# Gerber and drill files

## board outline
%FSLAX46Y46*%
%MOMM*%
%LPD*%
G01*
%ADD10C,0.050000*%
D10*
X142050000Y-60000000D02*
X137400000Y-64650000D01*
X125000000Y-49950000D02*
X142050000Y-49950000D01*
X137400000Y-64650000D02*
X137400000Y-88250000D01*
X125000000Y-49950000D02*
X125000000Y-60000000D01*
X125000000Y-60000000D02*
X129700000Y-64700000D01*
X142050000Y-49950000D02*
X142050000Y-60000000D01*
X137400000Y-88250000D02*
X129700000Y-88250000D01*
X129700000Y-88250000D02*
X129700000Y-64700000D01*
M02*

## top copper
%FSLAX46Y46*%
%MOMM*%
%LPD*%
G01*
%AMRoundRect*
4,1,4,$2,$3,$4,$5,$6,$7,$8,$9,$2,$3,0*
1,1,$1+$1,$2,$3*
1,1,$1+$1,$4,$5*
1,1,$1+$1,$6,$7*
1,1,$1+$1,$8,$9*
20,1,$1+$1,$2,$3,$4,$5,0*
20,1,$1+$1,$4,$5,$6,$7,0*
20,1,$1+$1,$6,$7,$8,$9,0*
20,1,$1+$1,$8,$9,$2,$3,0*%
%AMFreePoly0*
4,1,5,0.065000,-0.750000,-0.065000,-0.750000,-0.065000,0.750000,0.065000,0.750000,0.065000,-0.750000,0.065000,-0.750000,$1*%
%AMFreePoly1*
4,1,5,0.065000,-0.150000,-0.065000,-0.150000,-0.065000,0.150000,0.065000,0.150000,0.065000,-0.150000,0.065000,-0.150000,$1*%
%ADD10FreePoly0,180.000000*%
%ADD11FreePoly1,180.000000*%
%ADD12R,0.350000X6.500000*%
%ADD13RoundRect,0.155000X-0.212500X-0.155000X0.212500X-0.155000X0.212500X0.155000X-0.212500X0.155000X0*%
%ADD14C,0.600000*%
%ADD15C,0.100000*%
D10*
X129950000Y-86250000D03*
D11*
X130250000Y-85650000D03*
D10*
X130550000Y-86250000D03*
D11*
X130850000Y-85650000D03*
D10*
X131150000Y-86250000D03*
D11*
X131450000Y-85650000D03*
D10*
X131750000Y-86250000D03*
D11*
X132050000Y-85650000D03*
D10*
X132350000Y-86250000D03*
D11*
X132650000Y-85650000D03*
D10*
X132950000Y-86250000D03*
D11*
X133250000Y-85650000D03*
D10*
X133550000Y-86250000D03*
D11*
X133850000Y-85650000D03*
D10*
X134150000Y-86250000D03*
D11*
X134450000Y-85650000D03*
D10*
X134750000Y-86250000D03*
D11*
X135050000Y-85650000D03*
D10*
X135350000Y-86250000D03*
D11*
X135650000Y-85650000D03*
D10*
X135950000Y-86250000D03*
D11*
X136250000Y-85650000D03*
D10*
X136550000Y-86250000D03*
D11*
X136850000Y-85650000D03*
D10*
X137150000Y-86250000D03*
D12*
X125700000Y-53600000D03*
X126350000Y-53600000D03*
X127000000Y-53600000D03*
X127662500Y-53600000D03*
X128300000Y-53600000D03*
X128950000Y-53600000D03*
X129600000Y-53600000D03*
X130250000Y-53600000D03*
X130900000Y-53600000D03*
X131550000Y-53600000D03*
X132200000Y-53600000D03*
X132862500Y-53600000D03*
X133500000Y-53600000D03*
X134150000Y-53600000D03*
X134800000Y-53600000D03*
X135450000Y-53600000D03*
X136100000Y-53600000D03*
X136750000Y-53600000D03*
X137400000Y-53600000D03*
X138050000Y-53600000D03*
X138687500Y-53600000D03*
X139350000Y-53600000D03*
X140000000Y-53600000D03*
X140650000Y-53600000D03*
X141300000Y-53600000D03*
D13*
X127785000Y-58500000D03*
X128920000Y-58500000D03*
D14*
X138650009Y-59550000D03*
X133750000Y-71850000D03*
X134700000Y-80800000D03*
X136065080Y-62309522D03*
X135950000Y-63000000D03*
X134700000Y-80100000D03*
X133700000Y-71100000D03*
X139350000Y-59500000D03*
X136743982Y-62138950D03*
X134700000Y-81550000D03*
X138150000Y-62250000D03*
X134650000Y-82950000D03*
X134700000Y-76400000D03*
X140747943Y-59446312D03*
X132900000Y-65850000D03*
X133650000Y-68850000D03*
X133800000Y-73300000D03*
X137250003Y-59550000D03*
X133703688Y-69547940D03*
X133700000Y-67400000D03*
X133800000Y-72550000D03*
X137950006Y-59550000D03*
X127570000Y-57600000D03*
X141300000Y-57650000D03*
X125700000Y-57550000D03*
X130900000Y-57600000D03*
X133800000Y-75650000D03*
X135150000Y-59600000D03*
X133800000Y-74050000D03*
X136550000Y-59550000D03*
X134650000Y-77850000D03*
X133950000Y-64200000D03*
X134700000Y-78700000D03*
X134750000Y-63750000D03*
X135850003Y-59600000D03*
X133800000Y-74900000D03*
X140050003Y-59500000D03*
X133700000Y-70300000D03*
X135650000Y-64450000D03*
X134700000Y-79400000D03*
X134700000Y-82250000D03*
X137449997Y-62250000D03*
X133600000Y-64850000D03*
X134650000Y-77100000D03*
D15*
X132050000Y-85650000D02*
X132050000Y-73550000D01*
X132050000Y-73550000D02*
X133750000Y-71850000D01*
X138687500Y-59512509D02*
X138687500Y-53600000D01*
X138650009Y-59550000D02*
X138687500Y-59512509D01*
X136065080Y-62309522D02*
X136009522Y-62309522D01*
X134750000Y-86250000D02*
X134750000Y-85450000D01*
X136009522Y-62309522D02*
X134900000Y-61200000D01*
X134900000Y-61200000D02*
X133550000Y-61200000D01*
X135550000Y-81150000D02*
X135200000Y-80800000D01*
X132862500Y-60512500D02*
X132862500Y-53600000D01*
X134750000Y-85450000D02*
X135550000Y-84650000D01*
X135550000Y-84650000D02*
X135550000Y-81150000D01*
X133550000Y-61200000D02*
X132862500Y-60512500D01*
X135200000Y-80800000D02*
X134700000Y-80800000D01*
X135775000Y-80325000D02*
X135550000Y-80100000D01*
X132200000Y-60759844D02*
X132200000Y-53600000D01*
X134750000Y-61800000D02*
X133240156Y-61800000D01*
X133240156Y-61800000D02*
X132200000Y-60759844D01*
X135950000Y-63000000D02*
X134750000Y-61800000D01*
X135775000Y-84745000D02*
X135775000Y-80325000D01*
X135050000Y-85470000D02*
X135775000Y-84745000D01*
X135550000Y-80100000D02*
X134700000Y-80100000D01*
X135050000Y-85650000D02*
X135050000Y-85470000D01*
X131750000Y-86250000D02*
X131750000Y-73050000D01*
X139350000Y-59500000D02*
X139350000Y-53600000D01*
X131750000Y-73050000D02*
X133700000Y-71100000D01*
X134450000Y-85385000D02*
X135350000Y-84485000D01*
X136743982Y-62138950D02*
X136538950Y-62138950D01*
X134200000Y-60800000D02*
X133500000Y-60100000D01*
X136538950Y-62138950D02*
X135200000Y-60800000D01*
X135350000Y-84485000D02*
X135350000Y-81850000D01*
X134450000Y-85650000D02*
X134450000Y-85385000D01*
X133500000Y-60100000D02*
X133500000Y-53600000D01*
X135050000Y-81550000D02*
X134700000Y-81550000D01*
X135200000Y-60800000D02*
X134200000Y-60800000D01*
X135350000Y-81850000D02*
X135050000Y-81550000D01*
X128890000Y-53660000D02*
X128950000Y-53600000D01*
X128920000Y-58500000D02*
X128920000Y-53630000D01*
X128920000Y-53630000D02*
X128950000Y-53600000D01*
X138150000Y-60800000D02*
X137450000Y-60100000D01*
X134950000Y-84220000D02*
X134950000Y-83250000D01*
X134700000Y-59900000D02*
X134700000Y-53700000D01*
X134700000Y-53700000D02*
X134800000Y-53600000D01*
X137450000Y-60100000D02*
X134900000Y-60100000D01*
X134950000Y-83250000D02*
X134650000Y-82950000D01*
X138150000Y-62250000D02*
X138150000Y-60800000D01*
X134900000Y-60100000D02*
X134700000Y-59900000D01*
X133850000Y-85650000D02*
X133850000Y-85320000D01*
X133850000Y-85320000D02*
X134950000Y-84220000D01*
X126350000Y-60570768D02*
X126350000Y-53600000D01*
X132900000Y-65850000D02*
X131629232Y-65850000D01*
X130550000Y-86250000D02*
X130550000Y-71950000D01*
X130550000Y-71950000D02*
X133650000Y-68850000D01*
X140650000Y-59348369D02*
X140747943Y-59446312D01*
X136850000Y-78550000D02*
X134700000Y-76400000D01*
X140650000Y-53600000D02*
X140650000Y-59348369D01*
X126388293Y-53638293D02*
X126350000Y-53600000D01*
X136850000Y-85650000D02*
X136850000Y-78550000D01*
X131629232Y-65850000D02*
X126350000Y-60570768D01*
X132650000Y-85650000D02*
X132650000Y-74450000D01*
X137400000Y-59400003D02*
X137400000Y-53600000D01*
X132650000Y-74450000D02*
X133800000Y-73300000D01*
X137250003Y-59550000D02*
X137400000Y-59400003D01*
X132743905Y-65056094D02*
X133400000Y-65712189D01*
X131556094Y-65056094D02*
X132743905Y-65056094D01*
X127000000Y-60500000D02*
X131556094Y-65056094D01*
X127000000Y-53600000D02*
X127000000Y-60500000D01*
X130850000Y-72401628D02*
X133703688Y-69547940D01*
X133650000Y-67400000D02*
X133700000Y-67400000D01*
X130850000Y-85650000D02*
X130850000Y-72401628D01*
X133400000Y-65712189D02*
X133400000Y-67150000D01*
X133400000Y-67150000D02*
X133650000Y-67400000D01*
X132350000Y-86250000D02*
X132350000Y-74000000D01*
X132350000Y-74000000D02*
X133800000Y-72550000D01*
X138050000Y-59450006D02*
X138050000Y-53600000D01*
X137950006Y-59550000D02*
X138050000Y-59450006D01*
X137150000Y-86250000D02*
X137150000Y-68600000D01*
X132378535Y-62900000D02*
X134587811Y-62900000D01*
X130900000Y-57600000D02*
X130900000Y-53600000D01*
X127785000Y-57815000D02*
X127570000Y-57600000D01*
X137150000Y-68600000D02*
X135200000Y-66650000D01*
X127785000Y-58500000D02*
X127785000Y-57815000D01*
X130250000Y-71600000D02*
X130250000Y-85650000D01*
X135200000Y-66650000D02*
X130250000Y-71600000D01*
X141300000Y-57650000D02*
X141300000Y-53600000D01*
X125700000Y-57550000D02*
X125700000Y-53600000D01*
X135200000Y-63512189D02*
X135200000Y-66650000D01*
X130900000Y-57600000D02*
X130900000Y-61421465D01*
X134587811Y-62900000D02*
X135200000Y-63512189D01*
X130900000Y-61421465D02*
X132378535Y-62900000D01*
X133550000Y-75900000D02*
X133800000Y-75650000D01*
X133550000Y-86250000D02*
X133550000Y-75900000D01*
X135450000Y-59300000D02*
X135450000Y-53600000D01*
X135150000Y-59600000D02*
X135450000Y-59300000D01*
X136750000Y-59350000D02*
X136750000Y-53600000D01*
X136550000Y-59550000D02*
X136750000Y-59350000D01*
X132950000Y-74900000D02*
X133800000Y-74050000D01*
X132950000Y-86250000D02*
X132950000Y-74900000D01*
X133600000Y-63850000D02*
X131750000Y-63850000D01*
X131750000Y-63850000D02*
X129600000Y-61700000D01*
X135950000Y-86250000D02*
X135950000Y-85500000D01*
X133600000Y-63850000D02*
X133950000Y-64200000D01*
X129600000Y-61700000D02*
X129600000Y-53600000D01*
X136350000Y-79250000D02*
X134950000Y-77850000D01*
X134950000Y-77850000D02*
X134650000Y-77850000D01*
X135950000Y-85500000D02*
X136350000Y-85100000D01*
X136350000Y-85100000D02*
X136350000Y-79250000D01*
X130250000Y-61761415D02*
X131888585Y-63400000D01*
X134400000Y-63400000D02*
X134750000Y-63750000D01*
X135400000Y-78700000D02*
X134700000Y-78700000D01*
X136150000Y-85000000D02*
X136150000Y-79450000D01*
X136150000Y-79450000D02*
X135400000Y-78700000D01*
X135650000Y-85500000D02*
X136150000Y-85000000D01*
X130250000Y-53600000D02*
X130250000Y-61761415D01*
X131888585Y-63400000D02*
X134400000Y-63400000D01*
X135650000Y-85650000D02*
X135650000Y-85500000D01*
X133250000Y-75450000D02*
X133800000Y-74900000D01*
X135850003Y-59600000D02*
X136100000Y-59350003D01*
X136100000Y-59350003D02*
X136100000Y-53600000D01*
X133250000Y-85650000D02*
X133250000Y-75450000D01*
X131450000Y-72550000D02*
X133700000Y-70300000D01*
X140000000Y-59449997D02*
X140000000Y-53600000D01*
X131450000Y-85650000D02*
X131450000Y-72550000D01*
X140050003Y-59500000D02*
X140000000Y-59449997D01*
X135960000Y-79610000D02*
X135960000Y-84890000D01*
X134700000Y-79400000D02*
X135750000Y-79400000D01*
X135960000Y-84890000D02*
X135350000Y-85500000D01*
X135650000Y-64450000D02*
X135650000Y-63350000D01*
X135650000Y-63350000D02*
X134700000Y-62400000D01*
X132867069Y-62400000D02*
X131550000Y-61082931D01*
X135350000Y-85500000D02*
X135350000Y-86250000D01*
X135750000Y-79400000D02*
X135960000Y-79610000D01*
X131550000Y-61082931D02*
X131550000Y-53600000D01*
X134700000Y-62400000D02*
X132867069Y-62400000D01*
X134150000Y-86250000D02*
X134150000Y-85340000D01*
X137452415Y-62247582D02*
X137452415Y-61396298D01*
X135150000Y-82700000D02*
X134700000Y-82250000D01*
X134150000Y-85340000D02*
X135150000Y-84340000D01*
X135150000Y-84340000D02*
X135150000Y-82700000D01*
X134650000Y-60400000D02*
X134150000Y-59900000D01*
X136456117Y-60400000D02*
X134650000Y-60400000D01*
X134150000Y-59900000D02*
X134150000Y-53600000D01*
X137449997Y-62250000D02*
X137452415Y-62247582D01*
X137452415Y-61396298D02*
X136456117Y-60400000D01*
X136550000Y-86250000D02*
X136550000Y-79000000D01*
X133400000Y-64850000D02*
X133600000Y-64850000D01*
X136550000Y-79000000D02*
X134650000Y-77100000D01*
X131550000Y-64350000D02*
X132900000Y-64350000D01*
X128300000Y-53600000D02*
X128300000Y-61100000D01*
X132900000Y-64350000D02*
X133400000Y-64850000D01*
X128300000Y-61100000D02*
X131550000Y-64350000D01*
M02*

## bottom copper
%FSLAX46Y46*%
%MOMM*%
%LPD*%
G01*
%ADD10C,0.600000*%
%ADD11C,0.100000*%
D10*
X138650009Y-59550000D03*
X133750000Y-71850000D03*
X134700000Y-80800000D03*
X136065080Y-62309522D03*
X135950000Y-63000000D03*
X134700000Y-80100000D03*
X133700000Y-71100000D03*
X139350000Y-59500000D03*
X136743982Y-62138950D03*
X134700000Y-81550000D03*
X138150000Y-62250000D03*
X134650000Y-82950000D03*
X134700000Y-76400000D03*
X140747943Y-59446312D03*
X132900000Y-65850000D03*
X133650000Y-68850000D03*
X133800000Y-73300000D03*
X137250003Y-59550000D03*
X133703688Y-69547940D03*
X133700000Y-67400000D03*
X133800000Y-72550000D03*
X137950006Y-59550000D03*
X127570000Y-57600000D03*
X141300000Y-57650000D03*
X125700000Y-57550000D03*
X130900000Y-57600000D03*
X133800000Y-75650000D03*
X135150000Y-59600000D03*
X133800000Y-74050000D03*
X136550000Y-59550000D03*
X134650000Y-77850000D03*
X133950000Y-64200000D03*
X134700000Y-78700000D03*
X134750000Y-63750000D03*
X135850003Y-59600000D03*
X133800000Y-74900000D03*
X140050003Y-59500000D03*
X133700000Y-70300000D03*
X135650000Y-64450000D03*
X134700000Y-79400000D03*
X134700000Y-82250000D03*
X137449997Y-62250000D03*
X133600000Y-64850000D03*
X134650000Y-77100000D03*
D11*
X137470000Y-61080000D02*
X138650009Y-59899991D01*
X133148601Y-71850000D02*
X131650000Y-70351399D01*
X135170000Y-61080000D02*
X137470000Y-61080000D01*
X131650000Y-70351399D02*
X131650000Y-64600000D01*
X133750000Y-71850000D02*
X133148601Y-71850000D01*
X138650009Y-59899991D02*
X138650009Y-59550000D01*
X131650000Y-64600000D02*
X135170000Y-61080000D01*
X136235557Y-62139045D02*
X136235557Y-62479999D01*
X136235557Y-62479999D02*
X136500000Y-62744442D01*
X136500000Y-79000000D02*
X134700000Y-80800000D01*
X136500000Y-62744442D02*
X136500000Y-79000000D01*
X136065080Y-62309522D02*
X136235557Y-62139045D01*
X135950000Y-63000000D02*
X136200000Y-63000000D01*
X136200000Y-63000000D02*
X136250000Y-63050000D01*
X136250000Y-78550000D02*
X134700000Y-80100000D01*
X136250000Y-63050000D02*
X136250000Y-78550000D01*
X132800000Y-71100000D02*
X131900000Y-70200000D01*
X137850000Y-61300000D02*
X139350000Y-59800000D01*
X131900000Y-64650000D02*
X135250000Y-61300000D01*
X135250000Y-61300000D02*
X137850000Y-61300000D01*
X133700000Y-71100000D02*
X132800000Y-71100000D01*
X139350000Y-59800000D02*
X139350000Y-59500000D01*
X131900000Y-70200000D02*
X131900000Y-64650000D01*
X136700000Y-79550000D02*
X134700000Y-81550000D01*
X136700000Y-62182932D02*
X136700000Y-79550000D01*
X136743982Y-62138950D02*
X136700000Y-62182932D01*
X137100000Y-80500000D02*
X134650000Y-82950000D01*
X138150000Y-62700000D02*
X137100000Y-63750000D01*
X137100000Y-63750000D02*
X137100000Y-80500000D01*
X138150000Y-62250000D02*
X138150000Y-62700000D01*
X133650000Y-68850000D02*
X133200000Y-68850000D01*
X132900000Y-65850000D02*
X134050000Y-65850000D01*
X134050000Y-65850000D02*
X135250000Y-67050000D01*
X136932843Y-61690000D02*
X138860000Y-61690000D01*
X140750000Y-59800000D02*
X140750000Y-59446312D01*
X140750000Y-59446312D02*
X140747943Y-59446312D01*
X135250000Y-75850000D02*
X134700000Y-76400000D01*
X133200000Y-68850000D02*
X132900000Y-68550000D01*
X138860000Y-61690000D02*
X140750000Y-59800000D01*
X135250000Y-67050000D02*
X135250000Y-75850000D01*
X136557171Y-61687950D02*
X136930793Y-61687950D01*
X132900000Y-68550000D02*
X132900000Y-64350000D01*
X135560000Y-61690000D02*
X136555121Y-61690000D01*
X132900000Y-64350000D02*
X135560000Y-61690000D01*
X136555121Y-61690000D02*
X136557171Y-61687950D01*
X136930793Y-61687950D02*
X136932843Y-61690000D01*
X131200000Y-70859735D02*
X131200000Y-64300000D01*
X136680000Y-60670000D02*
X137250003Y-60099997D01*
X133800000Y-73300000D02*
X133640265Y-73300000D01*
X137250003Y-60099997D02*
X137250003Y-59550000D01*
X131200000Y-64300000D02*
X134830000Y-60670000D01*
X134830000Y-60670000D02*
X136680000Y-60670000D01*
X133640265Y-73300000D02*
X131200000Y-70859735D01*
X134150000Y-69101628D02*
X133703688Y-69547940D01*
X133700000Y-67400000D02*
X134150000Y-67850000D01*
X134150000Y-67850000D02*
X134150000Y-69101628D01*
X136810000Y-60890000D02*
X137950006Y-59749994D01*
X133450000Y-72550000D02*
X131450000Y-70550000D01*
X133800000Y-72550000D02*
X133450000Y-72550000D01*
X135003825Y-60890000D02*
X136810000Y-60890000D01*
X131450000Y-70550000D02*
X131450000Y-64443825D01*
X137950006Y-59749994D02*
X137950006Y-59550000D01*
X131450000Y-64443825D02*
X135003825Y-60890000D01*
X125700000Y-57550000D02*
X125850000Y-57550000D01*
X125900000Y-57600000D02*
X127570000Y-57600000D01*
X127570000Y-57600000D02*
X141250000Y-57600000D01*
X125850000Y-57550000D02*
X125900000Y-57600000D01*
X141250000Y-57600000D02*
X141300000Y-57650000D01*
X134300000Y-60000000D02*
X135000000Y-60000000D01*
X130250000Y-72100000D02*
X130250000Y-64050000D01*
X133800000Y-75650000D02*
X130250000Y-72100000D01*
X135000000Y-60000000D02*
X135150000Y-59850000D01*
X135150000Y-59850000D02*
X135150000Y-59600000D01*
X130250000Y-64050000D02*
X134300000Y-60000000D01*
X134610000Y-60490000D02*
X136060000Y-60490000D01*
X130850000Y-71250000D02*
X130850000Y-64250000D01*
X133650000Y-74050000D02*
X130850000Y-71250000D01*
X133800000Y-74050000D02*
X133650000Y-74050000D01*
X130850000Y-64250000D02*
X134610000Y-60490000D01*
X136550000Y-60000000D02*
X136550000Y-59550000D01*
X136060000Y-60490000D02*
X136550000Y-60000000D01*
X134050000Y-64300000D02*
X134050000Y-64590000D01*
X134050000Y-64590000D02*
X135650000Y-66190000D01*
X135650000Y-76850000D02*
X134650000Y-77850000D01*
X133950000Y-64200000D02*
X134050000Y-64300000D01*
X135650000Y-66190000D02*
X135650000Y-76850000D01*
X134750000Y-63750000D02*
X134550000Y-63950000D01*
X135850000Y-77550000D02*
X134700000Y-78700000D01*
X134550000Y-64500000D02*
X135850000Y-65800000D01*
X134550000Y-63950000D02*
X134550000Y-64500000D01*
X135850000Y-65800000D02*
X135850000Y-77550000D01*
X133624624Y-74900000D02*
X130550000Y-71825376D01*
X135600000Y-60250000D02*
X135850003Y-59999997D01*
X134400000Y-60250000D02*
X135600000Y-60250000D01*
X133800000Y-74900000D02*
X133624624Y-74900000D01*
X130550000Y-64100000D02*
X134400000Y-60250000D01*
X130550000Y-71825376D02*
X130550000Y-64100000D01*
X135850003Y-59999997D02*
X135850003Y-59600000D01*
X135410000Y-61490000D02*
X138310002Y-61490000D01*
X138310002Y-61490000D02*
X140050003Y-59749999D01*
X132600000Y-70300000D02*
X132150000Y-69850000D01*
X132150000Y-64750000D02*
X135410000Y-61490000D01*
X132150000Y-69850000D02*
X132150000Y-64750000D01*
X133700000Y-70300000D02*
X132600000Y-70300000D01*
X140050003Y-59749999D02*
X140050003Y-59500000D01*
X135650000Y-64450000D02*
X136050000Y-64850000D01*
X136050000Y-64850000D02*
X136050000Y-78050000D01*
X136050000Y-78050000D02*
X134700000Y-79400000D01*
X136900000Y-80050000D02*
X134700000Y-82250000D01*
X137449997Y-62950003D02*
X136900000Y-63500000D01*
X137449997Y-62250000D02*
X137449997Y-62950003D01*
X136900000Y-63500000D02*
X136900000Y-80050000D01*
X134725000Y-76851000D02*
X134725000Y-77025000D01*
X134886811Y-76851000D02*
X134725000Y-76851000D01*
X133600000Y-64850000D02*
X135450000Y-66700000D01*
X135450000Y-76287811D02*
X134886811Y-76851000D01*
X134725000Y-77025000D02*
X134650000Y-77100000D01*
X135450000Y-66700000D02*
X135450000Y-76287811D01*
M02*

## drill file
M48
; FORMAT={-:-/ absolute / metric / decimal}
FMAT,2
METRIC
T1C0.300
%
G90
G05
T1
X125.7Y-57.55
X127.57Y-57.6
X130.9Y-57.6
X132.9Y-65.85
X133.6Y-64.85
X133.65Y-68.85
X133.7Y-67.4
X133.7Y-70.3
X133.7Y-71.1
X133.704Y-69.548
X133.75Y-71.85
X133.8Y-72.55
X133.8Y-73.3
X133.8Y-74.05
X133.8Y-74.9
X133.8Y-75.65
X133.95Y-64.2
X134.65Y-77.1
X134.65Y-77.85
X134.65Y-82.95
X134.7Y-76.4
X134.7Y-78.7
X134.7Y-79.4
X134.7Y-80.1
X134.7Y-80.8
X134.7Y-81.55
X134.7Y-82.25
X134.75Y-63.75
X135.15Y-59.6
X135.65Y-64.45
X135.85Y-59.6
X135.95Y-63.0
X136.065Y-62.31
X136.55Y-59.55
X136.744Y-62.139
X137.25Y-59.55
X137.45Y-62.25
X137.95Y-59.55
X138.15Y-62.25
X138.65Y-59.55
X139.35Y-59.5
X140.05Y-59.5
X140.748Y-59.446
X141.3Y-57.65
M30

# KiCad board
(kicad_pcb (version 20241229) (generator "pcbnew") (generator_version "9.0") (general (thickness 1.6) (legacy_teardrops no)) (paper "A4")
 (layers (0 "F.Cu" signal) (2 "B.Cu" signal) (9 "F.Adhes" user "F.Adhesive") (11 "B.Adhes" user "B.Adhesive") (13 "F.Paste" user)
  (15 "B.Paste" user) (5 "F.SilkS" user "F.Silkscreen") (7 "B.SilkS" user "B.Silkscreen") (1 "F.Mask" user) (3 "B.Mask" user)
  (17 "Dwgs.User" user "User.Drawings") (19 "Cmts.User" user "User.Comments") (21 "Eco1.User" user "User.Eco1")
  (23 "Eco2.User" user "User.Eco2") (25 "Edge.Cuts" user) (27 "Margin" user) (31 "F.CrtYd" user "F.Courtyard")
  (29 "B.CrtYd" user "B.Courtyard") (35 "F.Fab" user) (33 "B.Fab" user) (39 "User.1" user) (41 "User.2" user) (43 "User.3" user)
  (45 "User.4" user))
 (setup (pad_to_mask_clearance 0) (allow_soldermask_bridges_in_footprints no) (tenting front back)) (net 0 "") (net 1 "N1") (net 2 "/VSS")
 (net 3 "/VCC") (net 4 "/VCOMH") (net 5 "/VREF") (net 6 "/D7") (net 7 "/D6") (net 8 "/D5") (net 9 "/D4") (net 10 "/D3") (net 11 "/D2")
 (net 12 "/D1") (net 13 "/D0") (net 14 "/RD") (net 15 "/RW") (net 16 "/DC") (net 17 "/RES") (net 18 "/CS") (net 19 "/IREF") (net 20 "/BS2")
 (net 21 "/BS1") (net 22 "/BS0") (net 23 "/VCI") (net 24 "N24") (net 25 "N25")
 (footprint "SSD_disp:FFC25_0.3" (layer "F.Cu") (at 137.15 86.25 180)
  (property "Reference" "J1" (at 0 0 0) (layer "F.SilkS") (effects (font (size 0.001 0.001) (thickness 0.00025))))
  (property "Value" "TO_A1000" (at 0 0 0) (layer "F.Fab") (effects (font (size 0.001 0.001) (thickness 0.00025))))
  (pad "1" smd custom (at 7.2 0 180) (size 0.13 1.5) (layers "F.Cu" "F.Mask" "F.Paste") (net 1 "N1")
   (options (clearance outline) (anchor rect)) (primitives))
  (pad "2" smd custom (at 6.9 0.6 180) (size 0.13 0.3) (layers "F.Cu" "F.Mask" "F.Paste") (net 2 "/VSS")
   (options (clearance outline) (anchor rect)) (primitives))
  (pad "3" smd custom (at 6.6 0 180) (size 0.13 1.5) (layers "F.Cu" "F.Mask" "F.Paste") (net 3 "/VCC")
   (options (clearance outline) (anchor rect)) (primitives))
  (pad "4" smd custom (at 6.3 0.6 180) (size 0.13 0.3) (layers "F.Cu" "F.Mask" "F.Paste") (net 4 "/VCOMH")
   (options (clearance outline) (anchor rect)) (primitives))
  (pad "5" smd custom (at 6 0 180) (size 0.13 1.5) (layers "F.Cu" "F.Mask" "F.Paste") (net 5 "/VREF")
   (options (clearance outline) (anchor rect)) (primitives))
  (pad "6" smd custom (at 5.7 0.6 180) (size 0.13 0.3) (layers "F.Cu" "F.Mask" "F.Paste") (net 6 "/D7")
   (options (clearance outline) (anchor rect)) (primitives))
  (pad "7" smd custom (at 5.4 0 180) (size 0.13 1.5) (layers "F.Cu" "F.Mask" "F.Paste") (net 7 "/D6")
   (options (clearance outline) (anchor rect)) (primitives))
  (pad "8" smd custom (at 5.1 0.6 180) (size 0.13 0.3) (layers "F.Cu" "F.Mask" "F.Paste") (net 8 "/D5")
   (options (clearance outline) (anchor rect)) (primitives))
  (pad "9" smd custom (at 4.8 0 180) (size 0.13 1.5) (layers "F.Cu" "F.Mask" "F.Paste") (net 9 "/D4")
   (options (clearance outline) (anchor rect)) (primitives))
  (pad "10" smd custom (at 4.5 0.6 180) (size 0.13 0.3) (layers "F.Cu" "F.Mask" "F.Paste") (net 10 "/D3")
   (options (clearance outline) (anchor rect)) (primitives))
  (pad "11" smd custom (at 4.2 0 180) (size 0.13 1.5) (layers "F.Cu" "F.Mask" "F.Paste") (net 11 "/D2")
   (options (clearance outline) (anchor rect)) (primitives))
  (pad "12" smd custom (at 3.9 0.6 180) (size 0.13 0.3) (layers "F.Cu" "F.Mask" "F.Paste") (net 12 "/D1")
   (options (clearance outline) (anchor rect)) (primitives))
  (pad "13" smd custom (at 3.6 0 180) (size 0.13 1.5) (layers "F.Cu" "F.Mask" "F.Paste") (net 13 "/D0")
   (options (clearance outline) (anchor rect)) (primitives))
  (pad "14" smd custom (at 3.3 0.6 180) (size 0.13 0.3) (layers "F.Cu" "F.Mask" "F.Paste") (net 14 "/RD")
   (options (clearance outline) (anchor rect)) (primitives))
  (pad "15" smd custom (at 3 0 180) (size 0.13 1.5) (layers "F.Cu" "F.Mask" "F.Paste") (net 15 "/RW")
   (options (clearance outline) (anchor rect)) (primitives))
  (pad "16" smd custom (at 2.7 0.6 180) (size 0.13 0.3) (layers "F.Cu" "F.Mask" "F.Paste") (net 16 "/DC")
   (options (clearance outline) (anchor rect)) (primitives))
  (pad "17" smd custom (at 2.4 0 180) (size 0.13 1.5) (layers "F.Cu" "F.Mask" "F.Paste") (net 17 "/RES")
   (options (clearance outline) (anchor rect)) (primitives))
  (pad "18" smd custom (at 2.1 0.6 180) (size 0.13 0.3) (layers "F.Cu" "F.Mask" "F.Paste") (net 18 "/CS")
   (options (clearance outline) (anchor rect)) (primitives))
  (pad "19" smd custom (at 1.8 0 180) (size 0.13 1.5) (layers "F.Cu" "F.Mask" "F.Paste") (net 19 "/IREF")
   (options (clearance outline) (anchor rect)) (primitives))
  (pad "20" smd custom (at 1.5 0.6 180) (size 0.13 0.3) (layers "F.Cu" "F.Mask" "F.Paste") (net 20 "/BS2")
   (options (clearance outline) (anchor rect)) (primitives))
  (pad "21" smd custom (at 1.2 0 180) (size 0.13 1.5) (layers "F.Cu" "F.Mask" "F.Paste") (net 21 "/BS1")
   (options (clearance outline) (anchor rect)) (primitives))
  (pad "22" smd custom (at 0.9 0.6 180) (size 0.13 0.3) (layers "F.Cu" "F.Mask" "F.Paste") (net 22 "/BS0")
   (options (clearance outline) (anchor rect)) (primitives))
  (pad "23" smd custom (at 0.6 0 180) (size 0.13 1.5) (layers "F.Cu" "F.Mask" "F.Paste") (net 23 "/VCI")
   (options (clearance outline) (anchor rect)) (primitives))
  (pad "24" smd custom (at 0.3 0.6 180) (size 0.13 0.3) (layers "F.Cu" "F.Mask" "F.Paste") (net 3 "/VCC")
   (options (clearance outline) (anchor rect)) (primitives))
  (pad "25" smd custom (at 0 0 180) (size 0.13 1.5) (layers "F.Cu" "F.Mask" "F.Paste") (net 2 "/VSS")
   (options (clearance outline) (anchor rect)) (primitives)))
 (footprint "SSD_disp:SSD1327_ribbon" (layer "F.Cu") (at 135.85 51.35)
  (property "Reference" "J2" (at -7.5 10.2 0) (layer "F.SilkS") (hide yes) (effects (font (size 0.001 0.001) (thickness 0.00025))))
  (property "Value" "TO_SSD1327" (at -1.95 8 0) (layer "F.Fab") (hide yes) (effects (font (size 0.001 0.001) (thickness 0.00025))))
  (pad "1" smd rect (at -10.15 2.25) (size 0.35 6.5) (layers "F.Cu" "F.Mask" "F.Paste") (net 2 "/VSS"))
  (pad "2" smd rect (at -9.5 2.25) (size 0.35 6.5) (layers "F.Cu" "F.Mask" "F.Paste") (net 3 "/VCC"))
  (pad "3" smd rect (at -8.85 2.25) (size 0.35 6.5) (layers "F.Cu" "F.Mask" "F.Paste") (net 4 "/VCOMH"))
  (pad "4" smd rect (at -8.1875 2.25) (size 0.35 6.5) (layers "F.Cu" "F.Mask" "F.Paste") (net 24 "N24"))
  (pad "5" smd rect (at -7.55 2.25) (size 0.35 6.5) (layers "F.Cu" "F.Mask" "F.Paste") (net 23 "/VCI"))
  (pad "6" smd rect (at -6.9 2.25) (size 0.35 6.5) (layers "F.Cu" "F.Mask" "F.Paste") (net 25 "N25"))
  (pad "7" smd rect (at -6.25 2.25) (size 0.35 6.5) (layers "F.Cu" "F.Mask" "F.Paste") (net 21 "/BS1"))
  (pad "8" smd rect (at -5.6 2.25) (size 0.35 6.5) (layers "F.Cu" "F.Mask" "F.Paste") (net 20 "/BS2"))
  (pad "9" smd rect (at -4.95 2.25) (size 0.35 6.5) (layers "F.Cu" "F.Mask" "F.Paste") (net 2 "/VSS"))
  (pad "10" smd rect (at -4.3 2.25) (size 0.35 6.5) (layers "F.Cu" "F.Mask" "F.Paste") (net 19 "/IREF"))
  (pad "11" smd rect (at -3.65 2.25) (size 0.35 6.5) (layers "F.Cu" "F.Mask" "F.Paste") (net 18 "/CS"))
  (pad "12" smd rect (at -2.9875 2.25) (size 0.35 6.5) (layers "F.Cu" "F.Mask" "F.Paste") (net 17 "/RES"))
  (pad "13" smd rect (at -2.35 2.25) (size 0.35 6.5) (layers "F.Cu" "F.Mask" "F.Paste") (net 16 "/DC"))
  (pad "14" smd rect (at -1.7 2.25) (size 0.35 6.5) (layers "F.Cu" "F.Mask" "F.Paste") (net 15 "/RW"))
  (pad "15" smd rect (at -1.05 2.25) (size 0.35 6.5) (layers "F.Cu" "F.Mask" "F.Paste") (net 14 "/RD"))
  (pad "16" smd rect (at -0.4 2.25) (size 0.35 6.5) (layers "F.Cu" "F.Mask" "F.Paste") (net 13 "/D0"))
  (pad "17" smd rect (at 0.25 2.25) (size 0.35 6.5) (layers "F.Cu" "F.Mask" "F.Paste") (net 12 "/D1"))
  (pad "18" smd rect (at 0.9 2.25) (size 0.35 6.5) (layers "F.Cu" "F.Mask" "F.Paste") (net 11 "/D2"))
  (pad "19" smd rect (at 1.55 2.25) (size 0.35 6.5) (layers "F.Cu" "F.Mask" "F.Paste") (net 10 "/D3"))
  (pad "20" smd rect (at 2.2 2.25) (size 0.35 6.5) (layers "F.Cu" "F.Mask" "F.Paste") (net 9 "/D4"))
  (pad "21" smd rect (at 2.8375 2.25) (size 0.35 6.5) (layers "F.Cu" "F.Mask" "F.Paste") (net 8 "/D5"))
  (pad "22" smd rect (at 3.5 2.25) (size 0.35 6.5) (layers "F.Cu" "F.Mask" "F.Paste") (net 7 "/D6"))
  (pad "23" smd rect (at 4.15 2.25) (size 0.35 6.5) (layers "F.Cu" "F.Mask" "F.Paste") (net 6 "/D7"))
  (pad "24" smd rect (at 4.8 2.25) (size 0.35 6.5) (layers "F.Cu" "F.Mask" "F.Paste") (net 3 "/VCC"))
  (pad "25" smd rect (at 5.45 2.25) (size 0.35 6.5) (layers "F.Cu" "F.Mask" "F.Paste") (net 2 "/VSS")))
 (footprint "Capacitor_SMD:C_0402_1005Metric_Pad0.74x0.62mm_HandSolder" (layer "F.Cu") (at 128.3525 58.5)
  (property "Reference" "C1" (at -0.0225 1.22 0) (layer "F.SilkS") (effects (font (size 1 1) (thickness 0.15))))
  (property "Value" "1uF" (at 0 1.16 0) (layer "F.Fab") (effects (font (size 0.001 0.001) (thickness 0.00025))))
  (pad "1" smd roundrect (at -0.5675 0) (size 0.735 0.62) (layers "F.Cu" "F.Mask" "F.Paste") (roundrect_rratio 0.25) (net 2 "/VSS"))
  (pad "2" smd roundrect (at 0.5675 0) (size 0.735 0.62) (layers "F.Cu" "F.Mask" "F.Paste") (roundrect_rratio 0.25) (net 25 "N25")))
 (gr_line (start 142.05 60) (end 137.4 64.65) (stroke (width 0.05) (type solid)) (layer "Edge.Cuts"))
 (gr_line (start 125 49.95) (end 142.05 49.95) (stroke (width 0.05) (type default)) (layer "Edge.Cuts"))
 (gr_line (start 137.4 64.65) (end 137.4 88.25) (stroke (width 0.05) (type solid)) (layer "Edge.Cuts"))
 (gr_line (start 125 49.95) (end 125 60) (stroke (width 0.05) (type solid)) (layer "Edge.Cuts"))
 (gr_line (start 125 60) (end 129.7 64.7) (stroke (width 0.05) (type solid)) (layer "Edge.Cuts"))
 (gr_line (start 142.05 49.95) (end 142.05 60) (stroke (width 0.05) (type solid)) (layer "Edge.Cuts"))
 (gr_line (start 137.4 88.25) (end 129.7 88.25) (stroke (width 0.05) (type default)) (layer "Edge.Cuts"))
 (gr_line (start 129.7 88.25) (end 129.7 64.7) (stroke (width 0.05) (type solid)) (layer "Edge.Cuts"))
 (segment (start 132.05 85.65) (end 132.05 73.55) (width 0.1) (layer "F.Cu") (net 8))
 (segment (start 132.05 73.55) (end 133.75 71.85) (width 0.1) (layer "F.Cu") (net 8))
 (segment (start 138.6875 59.512509) (end 138.6875 53.6) (width 0.1) (layer "F.Cu") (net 8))
 (segment (start 138.650009 59.55) (end 138.6875 59.512509) (width 0.1) (layer "F.Cu") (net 8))
 (via (at 138.650009 59.55) (size 0.6) (drill 0.3) (layers "F.Cu" "B.Cu") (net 8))
 (via (at 133.75 71.85) (size 0.6) (drill 0.3) (layers "F.Cu" "B.Cu") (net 8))
 (segment (start 137.47 61.08) (end 138.650009 59.899991) (width 0.1) (layer "B.Cu") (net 8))
 (segment (start 133.148601 71.85) (end 131.65 70.351399) (width 0.1) (layer "B.Cu") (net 8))
 (segment (start 135.17 61.08) (end 137.47 61.08) (width 0.1) (layer "B.Cu") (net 8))
 (segment (start 131.65 70.351399) (end 131.65 64.6) (width 0.1) (layer "B.Cu") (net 8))
 (segment (start 133.75 71.85) (end 133.148601 71.85) (width 0.1) (layer "B.Cu") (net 8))
 (segment (start 138.650009 59.899991) (end 138.650009 59.55) (width 0.1) (layer "B.Cu") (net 8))
 (segment (start 131.65 64.6) (end 135.17 61.08) (width 0.1) (layer "B.Cu") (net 8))
 (segment (start 136.06508 62.309522) (end 136.009522 62.309522) (width 0.1) (layer "F.Cu") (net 17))
 (segment (start 134.75 86.25) (end 134.75 85.45) (width 0.1) (layer "F.Cu") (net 17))
 (segment (start 136.009522 62.309522) (end 134.9 61.2) (width 0.1) (layer "F.Cu") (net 17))
 (segment (start 134.9 61.2) (end 133.55 61.2) (width 0.1) (layer "F.Cu") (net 17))
 (segment (start 135.55 81.15) (end 135.2 80.8) (width 0.1) (layer "F.Cu") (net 17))
 (segment (start 132.8625 60.5125) (end 132.8625 53.6) (width 0.1) (layer "F.Cu") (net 17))
 (segment (start 134.75 85.45) (end 135.55 84.65) (width 0.1) (layer "F.Cu") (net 17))
 (segment (start 135.55 84.65) (end 135.55 81.15) (width 0.1) (layer "F.Cu") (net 17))
 (segment (start 133.55 61.2) (end 132.8625 60.5125) (width 0.1) (layer "F.Cu") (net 17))
 (segment (start 135.2 80.8) (end 134.7 80.8) (width 0.1) (layer "F.Cu") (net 17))
 (via (at 134.7 80.8) (size 0.6) (drill 0.3) (layers "F.Cu" "B.Cu") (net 17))
 (via (at 136.06508 62.309522) (size 0.6) (drill 0.3) (layers "F.Cu" "B.Cu") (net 17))
 (segment (start 136.235557 62.139045) (end 136.235557 62.479999) (width 0.1) (layer "B.Cu") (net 17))
 (segment (start 136.235557 62.479999) (end 136.5 62.744442) (width 0.1) (layer "B.Cu") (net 17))
 (segment (start 136.5 79) (end 134.7 80.8) (width 0.1) (layer "B.Cu") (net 17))
 (segment (start 136.5 62.744442) (end 136.5 79) (width 0.1) (layer "B.Cu") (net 17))
 (segment (start 136.06508 62.309522) (end 136.235557 62.139045) (width 0.1) (layer "B.Cu") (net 17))
 (segment (start 135.775 80.325) (end 135.55 80.1) (width 0.1) (layer "F.Cu") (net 18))
 (segment (start 132.2 60.759844) (end 132.2 53.6) (width 0.1) (layer "F.Cu") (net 18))
 (segment (start 134.75 61.8) (end 133.240156 61.8) (width 0.1) (layer "F.Cu") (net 18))
 (segment (start 133.240156 61.8) (end 132.2 60.759844) (width 0.1) (layer "F.Cu") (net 18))
 (segment (start 135.95 63) (end 134.75 61.8) (width 0.1) (layer "F.Cu") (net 18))
 (segment (start 135.775 84.745) (end 135.775 80.325) (width 0.1) (layer "F.Cu") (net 18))
 (segment (start 135.05 85.47) (end 135.775 84.745) (width 0.1) (layer "F.Cu") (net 18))
 (segment (start 135.55 80.1) (end 134.7 80.1) (width 0.1) (layer "F.Cu") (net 18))
 (segment (start 135.05 85.65) (end 135.05 85.47) (width 0.1) (layer "F.Cu") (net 18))
 (via (at 135.95 63) (size 0.6) (drill 0.3) (layers "F.Cu" "B.Cu") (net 18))
 (via (at 134.7 80.1) (size 0.6) (drill 0.3) (layers "F.Cu" "B.Cu") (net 18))
 (segment (start 135.95 63) (end 136.2 63) (width 0.1) (layer "B.Cu") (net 18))
 (segment (start 136.2 63) (end 136.25 63.05) (width 0.1) (layer "B.Cu") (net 18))
 (segment (start 136.25 78.55) (end 134.7 80.1) (width 0.1) (layer "B.Cu") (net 18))
 (segment (start 136.25 63.05) (end 136.25 78.55) (width 0.1) (layer "B.Cu") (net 18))
 (segment (start 131.75 86.25) (end 131.75 73.05) (width 0.1) (layer "F.Cu") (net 7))
 (segment (start 139.35 59.5) (end 139.35 53.6) (width 0.1) (layer "F.Cu") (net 7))
 (segment (start 131.75 73.05) (end 133.7 71.1) (width 0.1) (layer "F.Cu") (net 7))
 (via (at 133.7 71.1) (size 0.6) (drill 0.3) (layers "F.Cu" "B.Cu") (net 7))
 (via (at 139.35 59.5) (size 0.6) (drill 0.3) (layers "F.Cu" "B.Cu") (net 7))
 (segment (start 132.8 71.1) (end 131.9 70.2) (width 0.1) (layer "B.Cu") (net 7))
 (segment (start 137.85 61.3) (end 139.35 59.8) (width 0.1) (layer "B.Cu") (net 7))
 (segment (start 131.9 64.65) (end 135.25 61.3) (width 0.1) (layer "B.Cu") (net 7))
 (segment (start 135.25 61.3) (end 137.85 61.3) (width 0.1) (layer "B.Cu") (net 7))
 (segment (start 133.7 71.1) (end 132.8 71.1) (width 0.1) (layer "B.Cu") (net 7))
 (segment (start 139.35 59.8) (end 139.35 59.5) (width 0.1) (layer "B.Cu") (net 7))
 (segment (start 131.9 70.2) (end 131.9 64.65) (width 0.1) (layer "B.Cu") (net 7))
 (segment (start 134.45 85.385) (end 135.35 84.485) (width 0.1) (layer "F.Cu") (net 16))
 (segment (start 136.743982 62.13895) (end 136.53895 62.13895) (width 0.1) (layer "F.Cu") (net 16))
 (segment (start 134.2 60.8) (end 133.5 60.1) (width 0.1) (layer "F.Cu") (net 16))
 (segment (start 136.53895 62.13895) (end 135.2 60.8) (width 0.1) (layer "F.Cu") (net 16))
 (segment (start 135.35 84.485) (end 135.35 81.85) (width 0.1) (layer "F.Cu") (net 16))
 (segment (start 134.45 85.65) (end 134.45 85.385) (width 0.1) (layer "F.Cu") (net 16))
 (segment (start 133.5 60.1) (end 133.5 53.6) (width 0.1) (layer "F.Cu") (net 16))
 (segment (start 135.05 81.55) (end 134.7 81.55) (width 0.1) (layer "F.Cu") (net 16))
 (segment (start 135.2 60.8) (end 134.2 60.8) (width 0.1) (layer "F.Cu") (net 16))
 (segment (start 135.35 81.85) (end 135.05 81.55) (width 0.1) (layer "F.Cu") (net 16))
 (via (at 136.743982 62.13895) (size 0.6) (drill 0.3) (layers "F.Cu" "B.Cu") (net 16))
 (via (at 134.7 81.55) (size 0.6) (drill 0.3) (layers "F.Cu" "B.Cu") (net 16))
 (segment (start 136.7 79.55) (end 134.7 81.55) (width 0.1) (layer "B.Cu") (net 16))
 (segment (start 136.7 62.182932) (end 136.7 79.55) (width 0.1) (layer "B.Cu") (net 16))
 (segment (start 136.743982 62.13895) (end 136.7 62.182932) (width 0.1) (layer "B.Cu") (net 16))
 (segment (start 128.89 53.66) (end 128.95 53.6) (width 0.1) (layer "F.Cu") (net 25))
 (segment (start 128.92 58.5) (end 128.92 53.63) (width 0.1) (layer "F.Cu") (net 25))
 (segment (start 128.92 53.63) (end 128.95 53.6) (width 0.1) (layer "F.Cu") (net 25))
 (segment (start 138.15 60.8) (end 137.45 60.1) (width 0.1) (layer "F.Cu") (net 14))
 (segment (start 134.95 84.22) (end 134.95 83.25) (width 0.1) (layer "F.Cu") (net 14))
 (segment (start 134.7 59.9) (end 134.7 53.7) (width 0.1) (layer "F.Cu") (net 14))
 (segment (start 134.7 53.7) (end 134.8 53.6) (width 0.1) (layer "F.Cu") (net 14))
 (segment (start 137.45 60.1) (end 134.9 60.1) (width 0.1) (layer "F.Cu") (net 14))
 (segment (start 134.95 83.25) (end 134.65 82.95) (width 0.1) (layer "F.Cu") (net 14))
 (segment (start 138.15 62.25) (end 138.15 60.8) (width 0.1) (layer "F.Cu") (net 14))
 (segment (start 134.9 60.1) (end 134.7 59.9) (width 0.1) (layer "F.Cu") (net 14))
 (segment (start 133.85 85.65) (end 133.85 85.32) (width 0.1) (layer "F.Cu") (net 14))
 (segment (start 133.85 85.32) (end 134.95 84.22) (width 0.1) (layer "F.Cu") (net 14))
 (via (at 138.15 62.25) (size 0.6) (drill 0.3) (layers "F.Cu" "B.Cu") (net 14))
 (via (at 134.65 82.95) (size 0.6) (drill 0.3) (layers "F.Cu" "B.Cu") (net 14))
 (segment (start 137.1 80.5) (end 134.65 82.95) (width 0.1) (layer "B.Cu") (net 14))
 (segment (start 138.15 62.7) (end 137.1 63.75) (width 0.1) (layer "B.Cu") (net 14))
 (segment (start 137.1 63.75) (end 137.1 80.5) (width 0.1) (layer "B.Cu") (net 14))
 (segment (start 138.15 62.25) (end 138.15 62.7) (width 0.1) (layer "B.Cu") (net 14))
 (segment (start 126.35 60.570768) (end 126.35 53.6) (width 0.1) (layer "F.Cu") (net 3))
 (segment (start 132.9 65.85) (end 131.629232 65.85) (width 0.1) (layer "F.Cu") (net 3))
 (segment (start 130.55 86.25) (end 130.55 71.95) (width 0.1) (layer "F.Cu") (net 3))
 (segment (start 130.55 71.95) (end 133.65 68.85) (width 0.1) (layer "F.Cu") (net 3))
 (segment (start 140.65 59.348369) (end 140.747943 59.446312) (width 0.1) (layer "F.Cu") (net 3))
 (segment (start 136.85 78.55) (end 134.7 76.4) (width 0.1) (layer "F.Cu") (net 3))
 (segment (start 140.65 53.6) (end 140.65 59.348369) (width 0.1) (layer "F.Cu") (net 3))
 (segment (start 126.388293 53.638293) (end 126.35 53.6) (width 0.1) (layer "F.Cu") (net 3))
 (segment (start 136.85 85.65) (end 136.85 78.55) (width 0.1) (layer "F.Cu") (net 3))
 (segment (start 131.629232 65.85) (end 126.35 60.570768) (width 0.1) (layer "F.Cu") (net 3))
 (via (at 134.7 76.4) (size 0.6) (drill 0.3) (layers "F.Cu" "B.Cu") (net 3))
 (via (at 140.747943 59.446312) (size 0.6) (drill 0.3) (layers "F.Cu" "B.Cu") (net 3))
 (via (at 132.9 65.85) (size 0.6) (drill 0.3) (layers "F.Cu" "B.Cu") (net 3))
 (via (at 133.65 68.85) (size 0.6) (drill 0.3) (layers "F.Cu" "B.Cu") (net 3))
 (segment (start 133.65 68.85) (end 133.2 68.85) (width 0.1) (layer "B.Cu") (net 3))
 (segment (start 132.9 65.85) (end 134.05 65.85) (width 0.1) (layer "B.Cu") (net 3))
 (segment (start 134.05 65.85) (end 135.25 67.05) (width 0.1) (layer "B.Cu") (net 3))
 (segment (start 136.932843 61.69) (end 138.86 61.69) (width 0.1) (layer "B.Cu") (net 3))
 (segment (start 140.75 59.8) (end 140.75 59.446312) (width 0.1) (layer "B.Cu") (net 3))
 (segment (start 140.75 59.446312) (end 140.747943 59.446312) (width 0.1) (layer "B.Cu") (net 3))
 (segment (start 135.25 75.85) (end 134.7 76.4) (width 0.1) (layer "B.Cu") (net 3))
 (segment (start 133.2 68.85) (end 132.9 68.55) (width 0.1) (layer "B.Cu") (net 3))
 (segment (start 138.86 61.69) (end 140.75 59.8) (width 0.1) (layer "B.Cu") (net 3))
 (segment (start 135.25 67.05) (end 135.25 75.85) (width 0.1) (layer "B.Cu") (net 3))
 (segment (start 136.557171 61.68795) (end 136.930793 61.68795) (width 0.1) (layer "B.Cu") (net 3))
 (segment (start 132.9 68.55) (end 132.9 64.35) (width 0.1) (layer "B.Cu") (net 3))
 (segment (start 135.56 61.69) (end 136.555121 61.69) (width 0.1) (layer "B.Cu") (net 3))
 (segment (start 132.9 64.35) (end 135.56 61.69) (width 0.1) (layer "B.Cu") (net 3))
 (segment (start 136.555121 61.69) (end 136.557171 61.68795) (width 0.1) (layer "B.Cu") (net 3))
 (segment (start 136.930793 61.68795) (end 136.932843 61.69) (width 0.1) (layer "B.Cu") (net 3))
 (segment (start 132.65 85.65) (end 132.65 74.45) (width 0.1) (layer "F.Cu") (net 10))
 (segment (start 137.4 59.400003) (end 137.4 53.6) (width 0.1) (layer "F.Cu") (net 10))
 (segment (start 132.65 74.45) (end 133.8 73.3) (width 0.1) (layer "F.Cu") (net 10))
 (segment (start 137.250003 59.55) (end 137.4 59.400003) (width 0.1) (layer "F.Cu") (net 10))
 (via (at 133.8 73.3) (size 0.6) (drill 0.3) (layers "F.Cu" "B.Cu") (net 10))
 (via (at 137.250003 59.55) (size 0.6) (drill 0.3) (layers "F.Cu" "B.Cu") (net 10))
 (segment (start 131.2 70.859735) (end 131.2 64.3) (width 0.1) (layer "B.Cu") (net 10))
 (segment (start 136.68 60.67) (end 137.250003 60.099997) (width 0.1) (layer "B.Cu") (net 10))
 (segment (start 133.8 73.3) (end 133.640265 73.3) (width 0.1) (layer "B.Cu") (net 10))
 (segment (start 137.250003 60.099997) (end 137.250003 59.55) (width 0.1) (layer "B.Cu") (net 10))
 (segment (start 131.2 64.3) (end 134.83 60.67) (width 0.1) (layer "B.Cu") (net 10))
 (segment (start 134.83 60.67) (end 136.68 60.67) (width 0.1) (layer "B.Cu") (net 10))
 (segment (start 133.640265 73.3) (end 131.2 70.859735) (width 0.1) (layer "B.Cu") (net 10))
 (segment (start 132.743905 65.056094) (end 133.4 65.712189) (width 0.1) (layer "F.Cu") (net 4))
 (segment (start 131.556094 65.056094) (end 132.743905 65.056094) (width 0.1) (layer "F.Cu") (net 4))
 (segment (start 127 60.5) (end 131.556094 65.056094) (width 0.1) (layer "F.Cu") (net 4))
 (segment (start 127 53.6) (end 127 60.5) (width 0.1) (layer "F.Cu") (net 4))
 (segment (start 130.85 72.401628) (end 133.703688 69.54794) (width 0.1) (layer "F.Cu") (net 4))
 (segment (start 133.65 67.4) (end 133.7 67.4) (width 0.1) (layer "F.Cu") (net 4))
 (segment (start 130.85 85.65) (end 130.85 72.401628) (width 0.1) (layer "F.Cu") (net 4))
 (segment (start 133.4 65.712189) (end 133.4 67.15) (width 0.1) (layer "F.Cu") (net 4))
 (segment (start 133.4 67.15) (end 133.65 67.4) (width 0.1) (layer "F.Cu") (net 4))
 (via (at 133.703688 69.54794) (size 0.6) (drill 0.3) (layers "F.Cu" "B.Cu") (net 4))
 (via (at 133.7 67.4) (size 0.6) (drill 0.3) (layers "F.Cu" "B.Cu") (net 4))
 (segment (start 134.15 69.101628) (end 133.703688 69.54794) (width 0.1) (layer "B.Cu") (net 4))
 (segment (start 133.7 67.4) (end 134.15 67.85) (width 0.1) (layer "B.Cu") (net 4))
 (segment (start 134.15 67.85) (end 134.15 69.101628) (width 0.1) (layer "B.Cu") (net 4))
 (segment (start 132.35 86.25) (end 132.35 74) (width 0.1) (layer "F.Cu") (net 9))
 (segment (start 132.35 74) (end 133.8 72.55) (width 0.1) (layer "F.Cu") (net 9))
 (segment (start 138.05 59.450006) (end 138.05 53.6) (width 0.1) (layer "F.Cu") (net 9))
 (segment (start 137.950006 59.55) (end 138.05 59.450006) (width 0.1) (layer "F.Cu") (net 9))
 (via (at 133.8 72.55) (size 0.6) (drill 0.3) (layers "F.Cu" "B.Cu") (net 9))
 (via (at 137.950006 59.55) (size 0.6) (drill 0.3) (layers "F.Cu" "B.Cu") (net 9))
 (segment (start 136.81 60.89) (end 137.950006 59.749994) (width 0.1) (layer "B.Cu") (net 9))
 (segment (start 133.45 72.55) (end 131.45 70.55) (width 0.1) (layer "B.Cu") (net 9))
 (segment (start 133.8 72.55) (end 133.45 72.55) (width 0.1) (layer "B.Cu") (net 9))
 (segment (start 135.003825 60.89) (end 136.81 60.89) (width 0.1) (layer "B.Cu") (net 9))
 (segment (start 131.45 70.55) (end 131.45 64.443825) (width 0.1) (layer "B.Cu") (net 9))
 (segment (start 137.950006 59.749994) (end 137.950006 59.55) (width 0.1) (layer "B.Cu") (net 9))
 (segment (start 131.45 64.443825) (end 135.003825 60.89) (width 0.1) (layer "B.Cu") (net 9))
 (segment (start 137.15 86.25) (end 137.15 68.6) (width 0.1) (layer "F.Cu") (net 2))
 (segment (start 132.378535 62.9) (end 134.587811 62.9) (width 0.1) (layer "F.Cu") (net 2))
 (segment (start 130.9 57.6) (end 130.9 53.6) (width 0.1) (layer "F.Cu") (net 2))
 (segment (start 127.785 57.815) (end 127.57 57.6) (width 0.1) (layer "F.Cu") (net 2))
 (segment (start 137.15 68.6) (end 135.2 66.65) (width 0.1) (layer "F.Cu") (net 2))
 (segment (start 127.785 58.5) (end 127.785 57.815) (width 0.1) (layer "F.Cu") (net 2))
 (segment (start 130.25 71.6) (end 130.25 85.65) (width 0.1) (layer "F.Cu") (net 2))
 (segment (start 135.2 66.65) (end 130.25 71.6) (width 0.1) (layer "F.Cu") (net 2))
 (segment (start 141.3 57.65) (end 141.3 53.6) (width 0.1) (layer "F.Cu") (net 2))
 (segment (start 125.7 57.55) (end 125.7 53.6) (width 0.1) (layer "F.Cu") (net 2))
 (segment (start 135.2 63.512189) (end 135.2 66.65) (width 0.1) (layer "F.Cu") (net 2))
 (segment (start 130.9 57.6) (end 130.9 61.421465) (width 0.1) (layer "F.Cu") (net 2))
 (segment (start 134.587811 62.9) (end 135.2 63.512189) (width 0.1) (layer "F.Cu") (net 2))
 (segment (start 130.9 61.421465) (end 132.378535 62.9) (width 0.1) (layer "F.Cu") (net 2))
 (via (at 127.57 57.6) (size 0.6) (drill 0.3) (layers "F.Cu" "B.Cu") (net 2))
 (via (at 141.3 57.65) (size 0.6) (drill 0.3) (layers "F.Cu" "B.Cu") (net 2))
 (via (at 125.7 57.55) (size 0.6) (drill 0.3) (layers "F.Cu" "B.Cu") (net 2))
 (via (at 130.9 57.6) (size 0.6) (drill 0.3) (layers "F.Cu" "B.Cu") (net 2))
 (segment (start 125.7 57.55) (end 125.85 57.55) (width 0.1) (layer "B.Cu") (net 2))
 (segment (start 125.9 57.6) (end 127.57 57.6) (width 0.1) (layer "B.Cu") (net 2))
 (segment (start 127.57 57.6) (end 141.25 57.6) (width 0.1) (layer "B.Cu") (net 2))
 (segment (start 125.85 57.55) (end 125.9 57.6) (width 0.1) (layer "B.Cu") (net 2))
 (segment (start 141.25 57.6) (end 141.3 57.65) (width 0.1) (layer "B.Cu") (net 2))
 (segment (start 133.55 75.9) (end 133.8 75.65) (width 0.1) (layer "F.Cu") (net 13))
 (segment (start 133.55 86.25) (end 133.55 75.9) (width 0.1) (layer "F.Cu") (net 13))
 (segment (start 135.45 59.3) (end 135.45 53.6) (width 0.1) (layer "F.Cu") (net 13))
 (segment (start 135.15 59.6) (end 135.45 59.3) (width 0.1) (layer "F.Cu") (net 13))
 (via (at 133.8 75.65) (size 0.6) (drill 0.3) (layers "F.Cu" "B.Cu") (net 13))
 (via (at 135.15 59.6) (size 0.6) (drill 0.3) (layers "F.Cu" "B.Cu") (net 13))
 (segment (start 134.3 60) (end 135 60) (width 0.1) (layer "B.Cu") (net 13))
 (segment (start 130.25 72.1) (end 130.25 64.05) (width 0.1) (layer "B.Cu") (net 13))
 (segment (start 133.8 75.65) (end 130.25 72.1) (width 0.1) (layer "B.Cu") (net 13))
 (segment (start 135 60) (end 135.15 59.85) (width 0.1) (layer "B.Cu") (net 13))
 (segment (start 135.15 59.85) (end 135.15 59.6) (width 0.1) (layer "B.Cu") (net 13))
 (segment (start 130.25 64.05) (end 134.3 60) (width 0.1) (layer "B.Cu") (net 13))
 (segment (start 136.75 59.35) (end 136.75 53.6) (width 0.1) (layer "F.Cu") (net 11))
 (segment (start 136.55 59.55) (end 136.75 59.35) (width 0.1) (layer "F.Cu") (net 11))
 (segment (start 132.95 74.9) (end 133.8 74.05) (width 0.1) (layer "F.Cu") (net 11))
 (segment (start 132.95 86.25) (end 132.95 74.9) (width 0.1) (layer "F.Cu") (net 11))
 (via (at 133.8 74.05) (size 0.6) (drill 0.3) (layers "F.Cu" "B.Cu") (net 11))
 (via (at 136.55 59.55) (size 0.6) (drill 0.3) (layers "F.Cu" "B.Cu") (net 11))
 (segment (start 134.61 60.49) (end 136.06 60.49) (width 0.1) (layer "B.Cu") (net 11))
 (segment (start 130.85 71.25) (end 130.85 64.25) (width 0.1) (layer "B.Cu") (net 11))
 (segment (start 133.65 74.05) (end 130.85 71.25) (width 0.1) (layer "B.Cu") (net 11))
 (segment (start 133.8 74.05) (end 133.65 74.05) (width 0.1) (layer "B.Cu") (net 11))
 (segment (start 130.85 64.25) (end 134.61 60.49) (width 0.1) (layer "B.Cu") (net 11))
 (segment (start 136.55 60) (end 136.55 59.55) (width 0.1) (layer "B.Cu") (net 11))
 (segment (start 136.06 60.49) (end 136.55 60) (width 0.1) (layer "B.Cu") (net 11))
 (segment (start 133.6 63.85) (end 131.75 63.85) (width 0.1) (layer "F.Cu") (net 21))
 (segment (start 131.75 63.85) (end 129.6 61.7) (width 0.1) (layer "F.Cu") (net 21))
 (segment (start 135.95 86.25) (end 135.95 85.5) (width 0.1) (layer "F.Cu") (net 21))
 (segment (start 133.6 63.85) (end 133.95 64.2) (width 0.1) (layer "F.Cu") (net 21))
 (segment (start 129.6 61.7) (end 129.6 53.6) (width 0.1) (layer "F.Cu") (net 21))
 (segment (start 136.35 79.25) (end 134.95 77.85) (width 0.1) (layer "F.Cu") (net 21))
 (segment (start 134.95 77.85) (end 134.65 77.85) (width 0.1) (layer "F.Cu") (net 21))
 (segment (start 135.95 85.5) (end 136.35 85.1) (width 0.1) (layer "F.Cu") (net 21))
 (segment (start 136.35 85.1) (end 136.35 79.25) (width 0.1) (layer "F.Cu") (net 21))
 (via (at 134.65 77.85) (size 0.6) (drill 0.3) (layers "F.Cu" "B.Cu") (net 21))
 (via (at 133.95 64.2) (size 0.6) (drill 0.3) (layers "F.Cu" "B.Cu") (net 21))
 (segment (start 134.05 64.3) (end 134.05 64.59) (width 0.1) (layer "B.Cu") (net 21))
 (segment (start 134.05 64.59) (end 135.65 66.19) (width 0.1) (layer "B.Cu") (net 21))
 (segment (start 135.65 76.85) (end 134.65 77.85) (width 0.1) (layer "B.Cu") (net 21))
 (segment (start 133.95 64.2) (end 134.05 64.3) (width 0.1) (layer "B.Cu") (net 21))
 (segment (start 135.65 66.19) (end 135.65 76.85) (width 0.1) (layer "B.Cu") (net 21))
 (segment (start 130.25 61.761415) (end 131.888585 63.4) (width 0.1) (layer "F.Cu") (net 20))
 (segment (start 134.4 63.4) (end 134.75 63.75) (width 0.1) (layer "F.Cu") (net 20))
 (segment (start 135.4 78.7) (end 134.7 78.7) (width 0.1) (layer "F.Cu") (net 20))
 (segment (start 136.15 85) (end 136.15 79.45) (width 0.1) (layer "F.Cu") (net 20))
 (segment (start 136.15 79.45) (end 135.4 78.7) (width 0.1) (layer "F.Cu") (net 20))
 (segment (start 135.65 85.5) (end 136.15 85) (width 0.1) (layer "F.Cu") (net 20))
 (segment (start 130.25 53.6) (end 130.25 61.761415) (width 0.1) (layer "F.Cu") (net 20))
 (segment (start 131.888585 63.4) (end 134.4 63.4) (width 0.1) (layer "F.Cu") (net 20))
 (segment (start 135.65 85.65) (end 135.65 85.5) (width 0.1) (layer "F.Cu") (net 20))
 (via (at 134.7 78.7) (size 0.6) (drill 0.3) (layers "F.Cu" "B.Cu") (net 20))
 (via (at 134.75 63.75) (size 0.6) (drill 0.3) (layers "F.Cu" "B.Cu") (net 20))
 (segment (start 134.75 63.75) (end 134.55 63.95) (width 0.1) (layer "B.Cu") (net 20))
 (segment (start 135.85 77.55) (end 134.7 78.7) (width 0.1) (layer "B.Cu") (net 20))
 (segment (start 134.55 64.5) (end 135.85 65.8) (width 0.1) (layer "B.Cu") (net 20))
 (segment (start 134.55 63.95) (end 134.55 64.5) (width 0.1) (layer "B.Cu") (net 20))
 (segment (start 135.85 65.8) (end 135.85 77.55) (width 0.1) (layer "B.Cu") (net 20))
 (segment (start 133.25 75.45) (end 133.8 74.9) (width 0.1) (layer "F.Cu") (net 12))
 (segment (start 135.850003 59.6) (end 136.1 59.350003) (width 0.1) (layer "F.Cu") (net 12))
 (segment (start 136.1 59.350003) (end 136.1 53.6) (width 0.1) (layer "F.Cu") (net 12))
 (segment (start 133.25 85.65) (end 133.25 75.45) (width 0.1) (layer "F.Cu") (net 12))
 (via (at 135.850003 59.6) (size 0.6) (drill 0.3) (layers "F.Cu" "B.Cu") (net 12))
 (via (at 133.8 74.9) (size 0.6) (drill 0.3) (layers "F.Cu" "B.Cu") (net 12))
 (segment (start 133.624624 74.9) (end 130.55 71.825376) (width 0.1) (layer "B.Cu") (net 12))
 (segment (start 135.6 60.25) (end 135.850003 59.999997) (width 0.1) (layer "B.Cu") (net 12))
 (segment (start 134.4 60.25) (end 135.6 60.25) (width 0.1) (layer "B.Cu") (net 12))
 (segment (start 133.8 74.9) (end 133.624624 74.9) (width 0.1) (layer "B.Cu") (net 12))
 (segment (start 130.55 64.1) (end 134.4 60.25) (width 0.1) (layer "B.Cu") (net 12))
 (segment (start 130.55 71.825376) (end 130.55 64.1) (width 0.1) (layer "B.Cu") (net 12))
 (segment (start 135.850003 59.999997) (end 135.850003 59.6) (width 0.1) (layer "B.Cu") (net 12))
 (segment (start 131.45 72.55) (end 133.7 70.3) (width 0.1) (layer "F.Cu") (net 6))
 (segment (start 140 59.449997) (end 140 53.6) (width 0.1) (layer "F.Cu") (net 6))
 (segment (start 131.45 85.65) (end 131.45 72.55) (width 0.1) (layer "F.Cu") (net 6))
 (segment (start 140.050003 59.5) (end 140 59.449997) (width 0.1) (layer "F.Cu") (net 6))
 (via (at 140.050003 59.5) (size 0.6) (drill 0.3) (layers "F.Cu" "B.Cu") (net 6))
 (via (at 133.7 70.3) (size 0.6) (drill 0.3) (layers "F.Cu" "B.Cu") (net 6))
 (segment (start 135.41 61.49) (end 138.310002 61.49) (width 0.1) (layer "B.Cu") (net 6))
 (segment (start 138.310002 61.49) (end 140.050003 59.749999) (width 0.1) (layer "B.Cu") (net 6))
 (segment (start 132.6 70.3) (end 132.15 69.85) (width 0.1) (layer "B.Cu") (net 6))
 (segment (start 132.15 64.75) (end 135.41 61.49) (width 0.1) (layer "B.Cu") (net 6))
 (segment (start 132.15 69.85) (end 132.15 64.75) (width 0.1) (layer "B.Cu") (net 6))
 (segment (start 133.7 70.3) (end 132.6 70.3) (width 0.1) (layer "B.Cu") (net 6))
 (segment (start 140.050003 59.749999) (end 140.050003 59.5) (width 0.1) (layer "B.Cu") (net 6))
 (segment (start 135.96 79.61) (end 135.96 84.89) (width 0.1) (layer "F.Cu") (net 19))
 (segment (start 134.7 79.4) (end 135.75 79.4) (width 0.1) (layer "F.Cu") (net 19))
 (segment (start 135.96 84.89) (end 135.35 85.5) (width 0.1) (layer "F.Cu") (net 19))
 (segment (start 135.65 64.45) (end 135.65 63.35) (width 0.1) (layer "F.Cu") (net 19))
 (segment (start 135.65 63.35) (end 134.7 62.4) (width 0.1) (layer "F.Cu") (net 19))
 (segment (start 132.867069 62.4) (end 131.55 61.082931) (width 0.1) (layer "F.Cu") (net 19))
 (segment (start 135.35 85.5) (end 135.35 86.25) (width 0.1) (layer "F.Cu") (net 19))
 (segment (start 135.75 79.4) (end 135.96 79.61) (width 0.1) (layer "F.Cu") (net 19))
 (segment (start 131.55 61.082931) (end 131.55 53.6) (width 0.1) (layer "F.Cu") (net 19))
 (segment (start 134.7 62.4) (end 132.867069 62.4) (width 0.1) (layer "F.Cu") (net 19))
 (via (at 135.65 64.45) (size 0.6) (drill 0.3) (layers "F.Cu" "B.Cu") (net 19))
 (via (at 134.7 79.4) (size 0.6) (drill 0.3) (layers "F.Cu" "B.Cu") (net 19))
 (segment (start 135.65 64.45) (end 136.05 64.85) (width 0.1) (layer "B.Cu") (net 19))
 (segment (start 136.05 64.85) (end 136.05 78.05) (width 0.1) (layer "B.Cu") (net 19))
 (segment (start 136.05 78.05) (end 134.7 79.4) (width 0.1) (layer "B.Cu") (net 19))
 (segment (start 134.15 86.25) (end 134.15 85.34) (width 0.1) (layer "F.Cu") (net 15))
 (segment (start 137.452415 62.247582) (end 137.452415 61.396298) (width 0.1) (layer "F.Cu") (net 15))
 (segment (start 135.15 82.7) (end 134.7 82.25) (width 0.1) (layer "F.Cu") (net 15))
 (segment (start 134.15 85.34) (end 135.15 84.34) (width 0.1) (layer "F.Cu") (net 15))
 (segment (start 135.15 84.34) (end 135.15 82.7) (width 0.1) (layer "F.Cu") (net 15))
 (segment (start 134.65 60.4) (end 134.15 59.9) (width 0.1) (layer "F.Cu") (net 15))
 (segment (start 136.456117 60.4) (end 134.65 60.4) (width 0.1) (layer "F.Cu") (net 15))
 (segment (start 134.15 59.9) (end 134.15 53.6) (width 0.1) (layer "F.Cu") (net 15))
 (segment (start 137.449997 62.25) (end 137.452415 62.247582) (width 0.1) (layer "F.Cu") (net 15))
 (segment (start 137.452415 61.396298) (end 136.456117 60.4) (width 0.1) (layer "F.Cu") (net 15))
 (via (at 134.7 82.25) (size 0.6) (drill 0.3) (layers "F.Cu" "B.Cu") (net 15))
 (via (at 137.449997 62.25) (size 0.6) (drill 0.3) (layers "F.Cu" "B.Cu") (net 15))
 (segment (start 136.9 80.05) (end 134.7 82.25) (width 0.1) (layer "B.Cu") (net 15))
 (segment (start 137.449997 62.950003) (end 136.9 63.5) (width 0.1) (layer "B.Cu") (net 15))
 (segment (start 137.449997 62.25) (end 137.449997 62.950003) (width 0.1) (layer "B.Cu") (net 15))
 (segment (start 136.9 63.5) (end 136.9 80.05) (width 0.1) (layer "B.Cu") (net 15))
 (segment (start 136.55 86.25) (end 136.55 79) (width 0.1) (layer "F.Cu") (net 23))
 (segment (start 133.4 64.85) (end 133.6 64.85) (width 0.1) (layer "F.Cu") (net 23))
 (segment (start 136.55 79) (end 134.65 77.1) (width 0.1) (layer "F.Cu") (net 23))
 (segment (start 131.55 64.35) (end 132.9 64.35) (width 0.1) (layer "F.Cu") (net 23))
 (segment (start 128.3 53.6) (end 128.3 61.1) (width 0.1) (layer "F.Cu") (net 23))
 (segment (start 132.9 64.35) (end 133.4 64.85) (width 0.1) (layer "F.Cu") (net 23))
 (segment (start 128.3 61.1) (end 131.55 64.35) (width 0.1) (layer "F.Cu") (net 23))
 (via (at 133.6 64.85) (size 0.6) (drill 0.3) (layers "F.Cu" "B.Cu") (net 23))
 (via (at 134.65 77.1) (size 0.6) (drill 0.3) (layers "F.Cu" "B.Cu") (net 23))
 (segment (start 134.725 76.851) (end 134.725 77.025) (width 0.1) (layer "B.Cu") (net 23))
 (segment (start 134.886811 76.851) (end 134.725 76.851) (width 0.1) (layer "B.Cu") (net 23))
 (segment (start 133.6 64.85) (end 135.45 66.7) (width 0.1) (layer "B.Cu") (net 23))
 (segment (start 135.45 76.287811) (end 134.886811 76.851) (width 0.1) (layer "B.Cu") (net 23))
 (segment (start 134.725 77.025) (end 134.65 77.1) (width 0.1) (layer "B.Cu") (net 23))
 (segment (start 135.45 66.7) (end 135.45 76.287811) (width 0.1) (layer "B.Cu") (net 23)))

